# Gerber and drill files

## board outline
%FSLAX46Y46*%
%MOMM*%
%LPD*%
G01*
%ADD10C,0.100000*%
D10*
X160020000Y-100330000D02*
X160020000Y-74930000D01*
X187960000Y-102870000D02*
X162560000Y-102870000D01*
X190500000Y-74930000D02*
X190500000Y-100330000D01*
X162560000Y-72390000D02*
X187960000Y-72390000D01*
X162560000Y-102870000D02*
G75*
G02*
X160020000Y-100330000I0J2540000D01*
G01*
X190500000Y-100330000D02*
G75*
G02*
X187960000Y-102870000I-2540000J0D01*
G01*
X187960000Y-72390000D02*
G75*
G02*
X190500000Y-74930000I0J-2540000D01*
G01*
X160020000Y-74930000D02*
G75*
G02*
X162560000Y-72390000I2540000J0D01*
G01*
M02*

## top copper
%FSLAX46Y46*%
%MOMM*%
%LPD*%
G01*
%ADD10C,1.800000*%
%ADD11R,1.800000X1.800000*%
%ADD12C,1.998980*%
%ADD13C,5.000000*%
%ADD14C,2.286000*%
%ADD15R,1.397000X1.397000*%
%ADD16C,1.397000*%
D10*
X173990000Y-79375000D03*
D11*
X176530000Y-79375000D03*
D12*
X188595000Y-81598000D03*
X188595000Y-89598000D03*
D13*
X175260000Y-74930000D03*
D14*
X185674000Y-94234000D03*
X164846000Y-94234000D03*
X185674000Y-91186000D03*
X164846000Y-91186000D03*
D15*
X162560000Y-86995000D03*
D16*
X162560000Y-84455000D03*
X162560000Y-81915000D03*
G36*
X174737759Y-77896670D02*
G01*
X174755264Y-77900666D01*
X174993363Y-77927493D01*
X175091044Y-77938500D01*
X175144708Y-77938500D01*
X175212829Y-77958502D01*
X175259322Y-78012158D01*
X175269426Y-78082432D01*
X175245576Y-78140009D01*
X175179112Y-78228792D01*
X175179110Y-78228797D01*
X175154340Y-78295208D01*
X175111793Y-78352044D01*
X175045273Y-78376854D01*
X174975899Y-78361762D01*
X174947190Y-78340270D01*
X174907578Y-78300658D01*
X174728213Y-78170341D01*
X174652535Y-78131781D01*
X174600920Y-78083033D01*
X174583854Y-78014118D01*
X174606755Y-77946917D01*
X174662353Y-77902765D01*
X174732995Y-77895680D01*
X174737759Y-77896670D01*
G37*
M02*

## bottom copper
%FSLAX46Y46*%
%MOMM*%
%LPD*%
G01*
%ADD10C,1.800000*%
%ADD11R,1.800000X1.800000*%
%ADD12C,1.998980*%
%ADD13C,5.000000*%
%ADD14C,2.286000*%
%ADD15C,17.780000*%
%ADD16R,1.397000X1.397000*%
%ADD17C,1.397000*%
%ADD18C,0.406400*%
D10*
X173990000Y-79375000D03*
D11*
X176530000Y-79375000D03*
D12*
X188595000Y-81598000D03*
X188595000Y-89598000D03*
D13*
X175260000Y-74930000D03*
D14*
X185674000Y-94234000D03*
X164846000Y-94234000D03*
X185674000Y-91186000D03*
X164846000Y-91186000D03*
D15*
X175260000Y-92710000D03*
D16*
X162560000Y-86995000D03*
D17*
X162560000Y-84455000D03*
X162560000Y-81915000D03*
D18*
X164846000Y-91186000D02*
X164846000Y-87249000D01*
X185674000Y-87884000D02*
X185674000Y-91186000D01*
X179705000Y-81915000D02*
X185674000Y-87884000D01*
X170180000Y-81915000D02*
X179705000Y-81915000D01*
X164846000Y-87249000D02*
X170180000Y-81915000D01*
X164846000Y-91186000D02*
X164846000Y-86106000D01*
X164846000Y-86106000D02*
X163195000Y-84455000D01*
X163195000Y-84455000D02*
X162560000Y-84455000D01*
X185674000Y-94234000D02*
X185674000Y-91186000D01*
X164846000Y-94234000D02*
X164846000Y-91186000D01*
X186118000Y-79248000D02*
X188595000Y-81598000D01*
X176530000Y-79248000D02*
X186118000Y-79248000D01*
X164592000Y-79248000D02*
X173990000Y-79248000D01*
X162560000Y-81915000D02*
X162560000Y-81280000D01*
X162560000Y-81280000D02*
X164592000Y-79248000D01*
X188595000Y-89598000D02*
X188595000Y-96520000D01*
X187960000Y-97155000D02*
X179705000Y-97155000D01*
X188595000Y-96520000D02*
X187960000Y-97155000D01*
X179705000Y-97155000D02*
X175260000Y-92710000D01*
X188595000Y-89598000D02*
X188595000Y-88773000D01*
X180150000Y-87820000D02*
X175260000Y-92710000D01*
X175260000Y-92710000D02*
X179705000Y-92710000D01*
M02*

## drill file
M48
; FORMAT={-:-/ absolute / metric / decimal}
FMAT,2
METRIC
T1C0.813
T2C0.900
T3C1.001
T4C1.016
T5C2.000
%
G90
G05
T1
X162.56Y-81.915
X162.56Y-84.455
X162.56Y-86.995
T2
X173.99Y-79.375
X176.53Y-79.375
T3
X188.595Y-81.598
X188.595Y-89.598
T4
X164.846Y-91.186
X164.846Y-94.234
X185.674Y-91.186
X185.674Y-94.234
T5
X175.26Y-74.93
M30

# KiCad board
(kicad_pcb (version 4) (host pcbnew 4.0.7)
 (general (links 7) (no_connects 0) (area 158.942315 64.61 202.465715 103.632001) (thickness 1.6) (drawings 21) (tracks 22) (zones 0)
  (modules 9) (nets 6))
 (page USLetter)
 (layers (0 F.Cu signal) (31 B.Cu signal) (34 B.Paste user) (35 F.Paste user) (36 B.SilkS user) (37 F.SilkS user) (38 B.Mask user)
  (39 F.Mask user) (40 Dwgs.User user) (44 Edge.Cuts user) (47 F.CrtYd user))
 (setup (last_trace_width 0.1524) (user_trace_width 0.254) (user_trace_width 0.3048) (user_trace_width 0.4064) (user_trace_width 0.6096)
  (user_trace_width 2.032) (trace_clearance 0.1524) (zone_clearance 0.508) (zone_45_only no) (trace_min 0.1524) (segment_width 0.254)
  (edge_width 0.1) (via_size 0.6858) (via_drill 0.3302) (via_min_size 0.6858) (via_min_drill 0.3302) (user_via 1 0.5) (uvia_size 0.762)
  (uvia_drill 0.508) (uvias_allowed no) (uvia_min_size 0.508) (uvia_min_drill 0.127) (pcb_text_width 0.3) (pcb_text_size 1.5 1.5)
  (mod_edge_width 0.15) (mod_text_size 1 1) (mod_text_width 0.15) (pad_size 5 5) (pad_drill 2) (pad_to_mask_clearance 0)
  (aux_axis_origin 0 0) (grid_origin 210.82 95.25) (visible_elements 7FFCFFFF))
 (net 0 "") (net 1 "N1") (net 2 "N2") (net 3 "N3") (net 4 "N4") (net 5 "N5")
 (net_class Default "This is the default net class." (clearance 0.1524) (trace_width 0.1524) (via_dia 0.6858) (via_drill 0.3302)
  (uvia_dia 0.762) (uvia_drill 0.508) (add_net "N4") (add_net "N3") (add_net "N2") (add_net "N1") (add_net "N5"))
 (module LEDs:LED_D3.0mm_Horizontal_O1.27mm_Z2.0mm (layer F.Cu) (at 173.99 79.375)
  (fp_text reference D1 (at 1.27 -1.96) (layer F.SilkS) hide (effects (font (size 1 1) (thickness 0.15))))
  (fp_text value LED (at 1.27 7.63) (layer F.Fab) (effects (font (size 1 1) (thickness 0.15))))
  (pad 2 thru_hole circle (at 0 0) (size 1.8 1.8) (drill 0.9) (layers *.Cu *.Mask) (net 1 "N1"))
  (pad 1 thru_hole rect (at 2.54 0) (size 1.8 1.8) (drill 0.9) (layers *.Cu *.Mask) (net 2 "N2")))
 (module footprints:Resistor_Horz (layer F.Cu) (at 188.595 85.598 270)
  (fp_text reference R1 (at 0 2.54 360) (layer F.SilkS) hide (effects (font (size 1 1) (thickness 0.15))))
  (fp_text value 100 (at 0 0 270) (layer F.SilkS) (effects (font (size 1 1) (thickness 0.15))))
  (pad 1 thru_hole circle (at -4 0 270) (size 1.99898 1.99898) (drill 1.00076) (layers *.Cu *.SilkS *.Mask) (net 2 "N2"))
  (pad 2 thru_hole circle (at 4 0 270) (size 1.99898 1.99898) (drill 1.00076) (layers *.Cu *.SilkS *.Mask) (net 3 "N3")))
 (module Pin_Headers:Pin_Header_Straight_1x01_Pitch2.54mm (layer F.Cu) (at 175.26 74.93)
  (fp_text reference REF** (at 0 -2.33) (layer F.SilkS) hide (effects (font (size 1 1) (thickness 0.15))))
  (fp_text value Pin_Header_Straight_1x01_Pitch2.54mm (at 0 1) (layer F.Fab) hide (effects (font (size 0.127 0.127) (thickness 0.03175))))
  (pad 1 thru_hole circle (at 0 0) (size 5 5) (drill 2) (layers *.Cu *.Mask)))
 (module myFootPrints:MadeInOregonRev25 (layer F.Cu) (at 167.64 76.454)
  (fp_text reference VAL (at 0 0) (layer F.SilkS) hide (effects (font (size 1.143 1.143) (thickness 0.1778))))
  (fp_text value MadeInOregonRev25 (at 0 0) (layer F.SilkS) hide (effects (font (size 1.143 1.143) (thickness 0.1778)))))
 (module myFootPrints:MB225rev (layer F.Cu) (at 184.15 76.2)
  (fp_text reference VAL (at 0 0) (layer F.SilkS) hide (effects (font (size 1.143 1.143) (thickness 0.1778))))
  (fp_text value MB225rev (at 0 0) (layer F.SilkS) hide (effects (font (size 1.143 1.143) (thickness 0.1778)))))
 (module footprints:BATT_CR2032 (layer B.Cu) (at 175.26 92.71 180)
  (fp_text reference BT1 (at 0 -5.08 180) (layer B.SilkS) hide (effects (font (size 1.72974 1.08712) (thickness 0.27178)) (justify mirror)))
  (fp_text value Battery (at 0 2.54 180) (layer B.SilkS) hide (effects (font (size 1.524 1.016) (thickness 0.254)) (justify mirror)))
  (pad 1 thru_hole circle (at -10.414 -1.524 180) (size 2.286 2.286) (drill 1.016) (layers *.Cu *.Mask B.SilkS) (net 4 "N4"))
  (pad 1 thru_hole circle (at 10.414 -1.524 180) (size 2.286 2.286) (drill 1.016) (layers *.Cu *.Mask B.SilkS) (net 4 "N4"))
  (pad 1 thru_hole circle (at -10.414 1.524 180) (size 2.286 2.286) (drill 1.016) (layers *.Cu *.Mask B.SilkS) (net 4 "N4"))
  (pad 1 thru_hole circle (at 10.414 1.524 180) (size 2.286 2.286) (drill 1.016) (layers *.Cu *.Mask B.SilkS) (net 4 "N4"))
  (pad 2 smd circle (at 0 0 180) (size 17.78 17.78) (layers B.Cu B.Paste B.Mask) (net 3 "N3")))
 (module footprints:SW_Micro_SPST (layer F.Cu) (at 162.56 84.455 90)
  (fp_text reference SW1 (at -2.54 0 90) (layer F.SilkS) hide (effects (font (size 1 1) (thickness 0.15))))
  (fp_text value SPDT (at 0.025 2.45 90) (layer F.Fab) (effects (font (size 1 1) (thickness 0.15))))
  (pad 1 thru_hole rect (at -2.54 0 90) (size 1.397 1.397) (drill 0.8128) (layers *.Cu *.Mask F.SilkS) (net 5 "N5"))
  (pad 2 thru_hole circle (at 0 0 90) (size 1.397 1.397) (drill 0.8128) (layers *.Cu *.Mask F.SilkS) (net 4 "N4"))
  (pad 3 thru_hole circle (at 2.54 0 90) (size 1.397 1.397) (drill 0.8128) (layers *.Cu *.Mask F.SilkS) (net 1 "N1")))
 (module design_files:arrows (layer F.Cu) (at 177.546 81.788)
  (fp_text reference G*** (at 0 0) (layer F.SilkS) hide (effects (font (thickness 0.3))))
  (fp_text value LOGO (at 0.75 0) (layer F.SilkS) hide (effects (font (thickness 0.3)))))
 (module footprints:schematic (layer F.Cu) (at 175.26 87.503)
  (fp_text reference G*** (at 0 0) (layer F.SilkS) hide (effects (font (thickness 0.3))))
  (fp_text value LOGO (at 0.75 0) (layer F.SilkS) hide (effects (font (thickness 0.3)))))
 (gr_line (start 160.02 100.33) (end 160.02 74.93) (angle 90) (layer Edge.Cuts) (width 0.1))
 (gr_line (start 187.96 102.87) (end 162.56 102.87) (angle 90) (layer Edge.Cuts) (width 0.1))
 (gr_line (start 190.5 74.93) (end 190.5 100.33) (angle 90) (layer Edge.Cuts) (width 0.1))
 (gr_line (start 162.56 72.39) (end 187.96 72.39) (angle 90) (layer Edge.Cuts) (width 0.1))
 (gr_arc (start 162.56 100.33) (end 162.56 102.87) (angle 90) (layer Edge.Cuts) (width 0.1))
 (gr_arc (start 187.96 100.33) (end 190.5 100.33) (angle 90) (layer Edge.Cuts) (width 0.1))
 (gr_arc (start 187.96 74.93) (end 187.96 72.39) (angle 90) (layer Edge.Cuts) (width 0.1))
 (gr_arc (start 162.56 74.93) (end 160.02 74.93) (angle 90) (layer Edge.Cuts) (width 0.1))
 (segment (start 164.846 91.186) (end 164.846 87.249) (width 0.4064) (layer B.Cu) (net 4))
 (segment (start 185.674 87.884) (end 185.674 91.186) (width 0.4064) (layer B.Cu) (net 4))
 (segment (start 179.705 81.915) (end 185.674 87.884) (width 0.4064) (layer B.Cu) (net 4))
 (segment (start 170.18 81.915) (end 179.705 81.915) (width 0.4064) (layer B.Cu) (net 4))
 (segment (start 164.846 87.249) (end 170.18 81.915) (width 0.4064) (layer B.Cu) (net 4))
 (segment (start 164.846 91.186) (end 164.846 86.106) (width 0.4064) (layer B.Cu) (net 4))
 (segment (start 164.846 86.106) (end 163.195 84.455) (width 0.4064) (layer B.Cu) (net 4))
 (segment (start 163.195 84.455) (end 162.56 84.455) (width 0.4064) (layer B.Cu) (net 4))
 (segment (start 185.674 94.234) (end 185.674 91.186) (width 0.4064) (layer B.Cu) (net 4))
 (segment (start 164.846 94.234) (end 164.846 91.186) (width 0.4064) (layer B.Cu) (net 4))
 (segment (start 186.118 79.248) (end 188.595 81.598) (width 0.4064) (layer B.Cu) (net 2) (status 20))
 (segment (start 176.53 79.248) (end 186.118 79.248) (width 0.4064) (layer B.Cu) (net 2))
 (segment (start 164.592 79.248) (end 173.99 79.248) (width 0.4064) (layer B.Cu) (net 1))
 (segment (start 162.56 81.915) (end 162.56 81.28) (width 0.4064) (layer B.Cu) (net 1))
 (segment (start 162.56 81.28) (end 164.592 79.248) (width 0.4064) (layer B.Cu) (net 1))
 (segment (start 188.595 89.598) (end 188.595 96.52) (width 0.4064) (layer B.Cu) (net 3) (status 10))
 (segment (start 187.96 97.155) (end 179.705 97.155) (width 0.4064) (layer B.Cu) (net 3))
 (segment (start 188.595 96.52) (end 187.96 97.155) (width 0.4064) (layer B.Cu) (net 3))
 (segment (start 179.705 97.155) (end 175.26 92.71) (width 0.4064) (layer B.Cu) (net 3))
 (segment (start 188.595 89.598) (end 188.595 88.773) (width 0.4064) (layer B.Cu) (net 3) (status 30))
 (segment (start 180.15 87.82) (end 175.26 92.71) (width 0.4064) (layer B.Cu) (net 3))
 (segment (start 175.26 92.71) (end 179.705 92.71) (width 0.4064) (layer B.Cu) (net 3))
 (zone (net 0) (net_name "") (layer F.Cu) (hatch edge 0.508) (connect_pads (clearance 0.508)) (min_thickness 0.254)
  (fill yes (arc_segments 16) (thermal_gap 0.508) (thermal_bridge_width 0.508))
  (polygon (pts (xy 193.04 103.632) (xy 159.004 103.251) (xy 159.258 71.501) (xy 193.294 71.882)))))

